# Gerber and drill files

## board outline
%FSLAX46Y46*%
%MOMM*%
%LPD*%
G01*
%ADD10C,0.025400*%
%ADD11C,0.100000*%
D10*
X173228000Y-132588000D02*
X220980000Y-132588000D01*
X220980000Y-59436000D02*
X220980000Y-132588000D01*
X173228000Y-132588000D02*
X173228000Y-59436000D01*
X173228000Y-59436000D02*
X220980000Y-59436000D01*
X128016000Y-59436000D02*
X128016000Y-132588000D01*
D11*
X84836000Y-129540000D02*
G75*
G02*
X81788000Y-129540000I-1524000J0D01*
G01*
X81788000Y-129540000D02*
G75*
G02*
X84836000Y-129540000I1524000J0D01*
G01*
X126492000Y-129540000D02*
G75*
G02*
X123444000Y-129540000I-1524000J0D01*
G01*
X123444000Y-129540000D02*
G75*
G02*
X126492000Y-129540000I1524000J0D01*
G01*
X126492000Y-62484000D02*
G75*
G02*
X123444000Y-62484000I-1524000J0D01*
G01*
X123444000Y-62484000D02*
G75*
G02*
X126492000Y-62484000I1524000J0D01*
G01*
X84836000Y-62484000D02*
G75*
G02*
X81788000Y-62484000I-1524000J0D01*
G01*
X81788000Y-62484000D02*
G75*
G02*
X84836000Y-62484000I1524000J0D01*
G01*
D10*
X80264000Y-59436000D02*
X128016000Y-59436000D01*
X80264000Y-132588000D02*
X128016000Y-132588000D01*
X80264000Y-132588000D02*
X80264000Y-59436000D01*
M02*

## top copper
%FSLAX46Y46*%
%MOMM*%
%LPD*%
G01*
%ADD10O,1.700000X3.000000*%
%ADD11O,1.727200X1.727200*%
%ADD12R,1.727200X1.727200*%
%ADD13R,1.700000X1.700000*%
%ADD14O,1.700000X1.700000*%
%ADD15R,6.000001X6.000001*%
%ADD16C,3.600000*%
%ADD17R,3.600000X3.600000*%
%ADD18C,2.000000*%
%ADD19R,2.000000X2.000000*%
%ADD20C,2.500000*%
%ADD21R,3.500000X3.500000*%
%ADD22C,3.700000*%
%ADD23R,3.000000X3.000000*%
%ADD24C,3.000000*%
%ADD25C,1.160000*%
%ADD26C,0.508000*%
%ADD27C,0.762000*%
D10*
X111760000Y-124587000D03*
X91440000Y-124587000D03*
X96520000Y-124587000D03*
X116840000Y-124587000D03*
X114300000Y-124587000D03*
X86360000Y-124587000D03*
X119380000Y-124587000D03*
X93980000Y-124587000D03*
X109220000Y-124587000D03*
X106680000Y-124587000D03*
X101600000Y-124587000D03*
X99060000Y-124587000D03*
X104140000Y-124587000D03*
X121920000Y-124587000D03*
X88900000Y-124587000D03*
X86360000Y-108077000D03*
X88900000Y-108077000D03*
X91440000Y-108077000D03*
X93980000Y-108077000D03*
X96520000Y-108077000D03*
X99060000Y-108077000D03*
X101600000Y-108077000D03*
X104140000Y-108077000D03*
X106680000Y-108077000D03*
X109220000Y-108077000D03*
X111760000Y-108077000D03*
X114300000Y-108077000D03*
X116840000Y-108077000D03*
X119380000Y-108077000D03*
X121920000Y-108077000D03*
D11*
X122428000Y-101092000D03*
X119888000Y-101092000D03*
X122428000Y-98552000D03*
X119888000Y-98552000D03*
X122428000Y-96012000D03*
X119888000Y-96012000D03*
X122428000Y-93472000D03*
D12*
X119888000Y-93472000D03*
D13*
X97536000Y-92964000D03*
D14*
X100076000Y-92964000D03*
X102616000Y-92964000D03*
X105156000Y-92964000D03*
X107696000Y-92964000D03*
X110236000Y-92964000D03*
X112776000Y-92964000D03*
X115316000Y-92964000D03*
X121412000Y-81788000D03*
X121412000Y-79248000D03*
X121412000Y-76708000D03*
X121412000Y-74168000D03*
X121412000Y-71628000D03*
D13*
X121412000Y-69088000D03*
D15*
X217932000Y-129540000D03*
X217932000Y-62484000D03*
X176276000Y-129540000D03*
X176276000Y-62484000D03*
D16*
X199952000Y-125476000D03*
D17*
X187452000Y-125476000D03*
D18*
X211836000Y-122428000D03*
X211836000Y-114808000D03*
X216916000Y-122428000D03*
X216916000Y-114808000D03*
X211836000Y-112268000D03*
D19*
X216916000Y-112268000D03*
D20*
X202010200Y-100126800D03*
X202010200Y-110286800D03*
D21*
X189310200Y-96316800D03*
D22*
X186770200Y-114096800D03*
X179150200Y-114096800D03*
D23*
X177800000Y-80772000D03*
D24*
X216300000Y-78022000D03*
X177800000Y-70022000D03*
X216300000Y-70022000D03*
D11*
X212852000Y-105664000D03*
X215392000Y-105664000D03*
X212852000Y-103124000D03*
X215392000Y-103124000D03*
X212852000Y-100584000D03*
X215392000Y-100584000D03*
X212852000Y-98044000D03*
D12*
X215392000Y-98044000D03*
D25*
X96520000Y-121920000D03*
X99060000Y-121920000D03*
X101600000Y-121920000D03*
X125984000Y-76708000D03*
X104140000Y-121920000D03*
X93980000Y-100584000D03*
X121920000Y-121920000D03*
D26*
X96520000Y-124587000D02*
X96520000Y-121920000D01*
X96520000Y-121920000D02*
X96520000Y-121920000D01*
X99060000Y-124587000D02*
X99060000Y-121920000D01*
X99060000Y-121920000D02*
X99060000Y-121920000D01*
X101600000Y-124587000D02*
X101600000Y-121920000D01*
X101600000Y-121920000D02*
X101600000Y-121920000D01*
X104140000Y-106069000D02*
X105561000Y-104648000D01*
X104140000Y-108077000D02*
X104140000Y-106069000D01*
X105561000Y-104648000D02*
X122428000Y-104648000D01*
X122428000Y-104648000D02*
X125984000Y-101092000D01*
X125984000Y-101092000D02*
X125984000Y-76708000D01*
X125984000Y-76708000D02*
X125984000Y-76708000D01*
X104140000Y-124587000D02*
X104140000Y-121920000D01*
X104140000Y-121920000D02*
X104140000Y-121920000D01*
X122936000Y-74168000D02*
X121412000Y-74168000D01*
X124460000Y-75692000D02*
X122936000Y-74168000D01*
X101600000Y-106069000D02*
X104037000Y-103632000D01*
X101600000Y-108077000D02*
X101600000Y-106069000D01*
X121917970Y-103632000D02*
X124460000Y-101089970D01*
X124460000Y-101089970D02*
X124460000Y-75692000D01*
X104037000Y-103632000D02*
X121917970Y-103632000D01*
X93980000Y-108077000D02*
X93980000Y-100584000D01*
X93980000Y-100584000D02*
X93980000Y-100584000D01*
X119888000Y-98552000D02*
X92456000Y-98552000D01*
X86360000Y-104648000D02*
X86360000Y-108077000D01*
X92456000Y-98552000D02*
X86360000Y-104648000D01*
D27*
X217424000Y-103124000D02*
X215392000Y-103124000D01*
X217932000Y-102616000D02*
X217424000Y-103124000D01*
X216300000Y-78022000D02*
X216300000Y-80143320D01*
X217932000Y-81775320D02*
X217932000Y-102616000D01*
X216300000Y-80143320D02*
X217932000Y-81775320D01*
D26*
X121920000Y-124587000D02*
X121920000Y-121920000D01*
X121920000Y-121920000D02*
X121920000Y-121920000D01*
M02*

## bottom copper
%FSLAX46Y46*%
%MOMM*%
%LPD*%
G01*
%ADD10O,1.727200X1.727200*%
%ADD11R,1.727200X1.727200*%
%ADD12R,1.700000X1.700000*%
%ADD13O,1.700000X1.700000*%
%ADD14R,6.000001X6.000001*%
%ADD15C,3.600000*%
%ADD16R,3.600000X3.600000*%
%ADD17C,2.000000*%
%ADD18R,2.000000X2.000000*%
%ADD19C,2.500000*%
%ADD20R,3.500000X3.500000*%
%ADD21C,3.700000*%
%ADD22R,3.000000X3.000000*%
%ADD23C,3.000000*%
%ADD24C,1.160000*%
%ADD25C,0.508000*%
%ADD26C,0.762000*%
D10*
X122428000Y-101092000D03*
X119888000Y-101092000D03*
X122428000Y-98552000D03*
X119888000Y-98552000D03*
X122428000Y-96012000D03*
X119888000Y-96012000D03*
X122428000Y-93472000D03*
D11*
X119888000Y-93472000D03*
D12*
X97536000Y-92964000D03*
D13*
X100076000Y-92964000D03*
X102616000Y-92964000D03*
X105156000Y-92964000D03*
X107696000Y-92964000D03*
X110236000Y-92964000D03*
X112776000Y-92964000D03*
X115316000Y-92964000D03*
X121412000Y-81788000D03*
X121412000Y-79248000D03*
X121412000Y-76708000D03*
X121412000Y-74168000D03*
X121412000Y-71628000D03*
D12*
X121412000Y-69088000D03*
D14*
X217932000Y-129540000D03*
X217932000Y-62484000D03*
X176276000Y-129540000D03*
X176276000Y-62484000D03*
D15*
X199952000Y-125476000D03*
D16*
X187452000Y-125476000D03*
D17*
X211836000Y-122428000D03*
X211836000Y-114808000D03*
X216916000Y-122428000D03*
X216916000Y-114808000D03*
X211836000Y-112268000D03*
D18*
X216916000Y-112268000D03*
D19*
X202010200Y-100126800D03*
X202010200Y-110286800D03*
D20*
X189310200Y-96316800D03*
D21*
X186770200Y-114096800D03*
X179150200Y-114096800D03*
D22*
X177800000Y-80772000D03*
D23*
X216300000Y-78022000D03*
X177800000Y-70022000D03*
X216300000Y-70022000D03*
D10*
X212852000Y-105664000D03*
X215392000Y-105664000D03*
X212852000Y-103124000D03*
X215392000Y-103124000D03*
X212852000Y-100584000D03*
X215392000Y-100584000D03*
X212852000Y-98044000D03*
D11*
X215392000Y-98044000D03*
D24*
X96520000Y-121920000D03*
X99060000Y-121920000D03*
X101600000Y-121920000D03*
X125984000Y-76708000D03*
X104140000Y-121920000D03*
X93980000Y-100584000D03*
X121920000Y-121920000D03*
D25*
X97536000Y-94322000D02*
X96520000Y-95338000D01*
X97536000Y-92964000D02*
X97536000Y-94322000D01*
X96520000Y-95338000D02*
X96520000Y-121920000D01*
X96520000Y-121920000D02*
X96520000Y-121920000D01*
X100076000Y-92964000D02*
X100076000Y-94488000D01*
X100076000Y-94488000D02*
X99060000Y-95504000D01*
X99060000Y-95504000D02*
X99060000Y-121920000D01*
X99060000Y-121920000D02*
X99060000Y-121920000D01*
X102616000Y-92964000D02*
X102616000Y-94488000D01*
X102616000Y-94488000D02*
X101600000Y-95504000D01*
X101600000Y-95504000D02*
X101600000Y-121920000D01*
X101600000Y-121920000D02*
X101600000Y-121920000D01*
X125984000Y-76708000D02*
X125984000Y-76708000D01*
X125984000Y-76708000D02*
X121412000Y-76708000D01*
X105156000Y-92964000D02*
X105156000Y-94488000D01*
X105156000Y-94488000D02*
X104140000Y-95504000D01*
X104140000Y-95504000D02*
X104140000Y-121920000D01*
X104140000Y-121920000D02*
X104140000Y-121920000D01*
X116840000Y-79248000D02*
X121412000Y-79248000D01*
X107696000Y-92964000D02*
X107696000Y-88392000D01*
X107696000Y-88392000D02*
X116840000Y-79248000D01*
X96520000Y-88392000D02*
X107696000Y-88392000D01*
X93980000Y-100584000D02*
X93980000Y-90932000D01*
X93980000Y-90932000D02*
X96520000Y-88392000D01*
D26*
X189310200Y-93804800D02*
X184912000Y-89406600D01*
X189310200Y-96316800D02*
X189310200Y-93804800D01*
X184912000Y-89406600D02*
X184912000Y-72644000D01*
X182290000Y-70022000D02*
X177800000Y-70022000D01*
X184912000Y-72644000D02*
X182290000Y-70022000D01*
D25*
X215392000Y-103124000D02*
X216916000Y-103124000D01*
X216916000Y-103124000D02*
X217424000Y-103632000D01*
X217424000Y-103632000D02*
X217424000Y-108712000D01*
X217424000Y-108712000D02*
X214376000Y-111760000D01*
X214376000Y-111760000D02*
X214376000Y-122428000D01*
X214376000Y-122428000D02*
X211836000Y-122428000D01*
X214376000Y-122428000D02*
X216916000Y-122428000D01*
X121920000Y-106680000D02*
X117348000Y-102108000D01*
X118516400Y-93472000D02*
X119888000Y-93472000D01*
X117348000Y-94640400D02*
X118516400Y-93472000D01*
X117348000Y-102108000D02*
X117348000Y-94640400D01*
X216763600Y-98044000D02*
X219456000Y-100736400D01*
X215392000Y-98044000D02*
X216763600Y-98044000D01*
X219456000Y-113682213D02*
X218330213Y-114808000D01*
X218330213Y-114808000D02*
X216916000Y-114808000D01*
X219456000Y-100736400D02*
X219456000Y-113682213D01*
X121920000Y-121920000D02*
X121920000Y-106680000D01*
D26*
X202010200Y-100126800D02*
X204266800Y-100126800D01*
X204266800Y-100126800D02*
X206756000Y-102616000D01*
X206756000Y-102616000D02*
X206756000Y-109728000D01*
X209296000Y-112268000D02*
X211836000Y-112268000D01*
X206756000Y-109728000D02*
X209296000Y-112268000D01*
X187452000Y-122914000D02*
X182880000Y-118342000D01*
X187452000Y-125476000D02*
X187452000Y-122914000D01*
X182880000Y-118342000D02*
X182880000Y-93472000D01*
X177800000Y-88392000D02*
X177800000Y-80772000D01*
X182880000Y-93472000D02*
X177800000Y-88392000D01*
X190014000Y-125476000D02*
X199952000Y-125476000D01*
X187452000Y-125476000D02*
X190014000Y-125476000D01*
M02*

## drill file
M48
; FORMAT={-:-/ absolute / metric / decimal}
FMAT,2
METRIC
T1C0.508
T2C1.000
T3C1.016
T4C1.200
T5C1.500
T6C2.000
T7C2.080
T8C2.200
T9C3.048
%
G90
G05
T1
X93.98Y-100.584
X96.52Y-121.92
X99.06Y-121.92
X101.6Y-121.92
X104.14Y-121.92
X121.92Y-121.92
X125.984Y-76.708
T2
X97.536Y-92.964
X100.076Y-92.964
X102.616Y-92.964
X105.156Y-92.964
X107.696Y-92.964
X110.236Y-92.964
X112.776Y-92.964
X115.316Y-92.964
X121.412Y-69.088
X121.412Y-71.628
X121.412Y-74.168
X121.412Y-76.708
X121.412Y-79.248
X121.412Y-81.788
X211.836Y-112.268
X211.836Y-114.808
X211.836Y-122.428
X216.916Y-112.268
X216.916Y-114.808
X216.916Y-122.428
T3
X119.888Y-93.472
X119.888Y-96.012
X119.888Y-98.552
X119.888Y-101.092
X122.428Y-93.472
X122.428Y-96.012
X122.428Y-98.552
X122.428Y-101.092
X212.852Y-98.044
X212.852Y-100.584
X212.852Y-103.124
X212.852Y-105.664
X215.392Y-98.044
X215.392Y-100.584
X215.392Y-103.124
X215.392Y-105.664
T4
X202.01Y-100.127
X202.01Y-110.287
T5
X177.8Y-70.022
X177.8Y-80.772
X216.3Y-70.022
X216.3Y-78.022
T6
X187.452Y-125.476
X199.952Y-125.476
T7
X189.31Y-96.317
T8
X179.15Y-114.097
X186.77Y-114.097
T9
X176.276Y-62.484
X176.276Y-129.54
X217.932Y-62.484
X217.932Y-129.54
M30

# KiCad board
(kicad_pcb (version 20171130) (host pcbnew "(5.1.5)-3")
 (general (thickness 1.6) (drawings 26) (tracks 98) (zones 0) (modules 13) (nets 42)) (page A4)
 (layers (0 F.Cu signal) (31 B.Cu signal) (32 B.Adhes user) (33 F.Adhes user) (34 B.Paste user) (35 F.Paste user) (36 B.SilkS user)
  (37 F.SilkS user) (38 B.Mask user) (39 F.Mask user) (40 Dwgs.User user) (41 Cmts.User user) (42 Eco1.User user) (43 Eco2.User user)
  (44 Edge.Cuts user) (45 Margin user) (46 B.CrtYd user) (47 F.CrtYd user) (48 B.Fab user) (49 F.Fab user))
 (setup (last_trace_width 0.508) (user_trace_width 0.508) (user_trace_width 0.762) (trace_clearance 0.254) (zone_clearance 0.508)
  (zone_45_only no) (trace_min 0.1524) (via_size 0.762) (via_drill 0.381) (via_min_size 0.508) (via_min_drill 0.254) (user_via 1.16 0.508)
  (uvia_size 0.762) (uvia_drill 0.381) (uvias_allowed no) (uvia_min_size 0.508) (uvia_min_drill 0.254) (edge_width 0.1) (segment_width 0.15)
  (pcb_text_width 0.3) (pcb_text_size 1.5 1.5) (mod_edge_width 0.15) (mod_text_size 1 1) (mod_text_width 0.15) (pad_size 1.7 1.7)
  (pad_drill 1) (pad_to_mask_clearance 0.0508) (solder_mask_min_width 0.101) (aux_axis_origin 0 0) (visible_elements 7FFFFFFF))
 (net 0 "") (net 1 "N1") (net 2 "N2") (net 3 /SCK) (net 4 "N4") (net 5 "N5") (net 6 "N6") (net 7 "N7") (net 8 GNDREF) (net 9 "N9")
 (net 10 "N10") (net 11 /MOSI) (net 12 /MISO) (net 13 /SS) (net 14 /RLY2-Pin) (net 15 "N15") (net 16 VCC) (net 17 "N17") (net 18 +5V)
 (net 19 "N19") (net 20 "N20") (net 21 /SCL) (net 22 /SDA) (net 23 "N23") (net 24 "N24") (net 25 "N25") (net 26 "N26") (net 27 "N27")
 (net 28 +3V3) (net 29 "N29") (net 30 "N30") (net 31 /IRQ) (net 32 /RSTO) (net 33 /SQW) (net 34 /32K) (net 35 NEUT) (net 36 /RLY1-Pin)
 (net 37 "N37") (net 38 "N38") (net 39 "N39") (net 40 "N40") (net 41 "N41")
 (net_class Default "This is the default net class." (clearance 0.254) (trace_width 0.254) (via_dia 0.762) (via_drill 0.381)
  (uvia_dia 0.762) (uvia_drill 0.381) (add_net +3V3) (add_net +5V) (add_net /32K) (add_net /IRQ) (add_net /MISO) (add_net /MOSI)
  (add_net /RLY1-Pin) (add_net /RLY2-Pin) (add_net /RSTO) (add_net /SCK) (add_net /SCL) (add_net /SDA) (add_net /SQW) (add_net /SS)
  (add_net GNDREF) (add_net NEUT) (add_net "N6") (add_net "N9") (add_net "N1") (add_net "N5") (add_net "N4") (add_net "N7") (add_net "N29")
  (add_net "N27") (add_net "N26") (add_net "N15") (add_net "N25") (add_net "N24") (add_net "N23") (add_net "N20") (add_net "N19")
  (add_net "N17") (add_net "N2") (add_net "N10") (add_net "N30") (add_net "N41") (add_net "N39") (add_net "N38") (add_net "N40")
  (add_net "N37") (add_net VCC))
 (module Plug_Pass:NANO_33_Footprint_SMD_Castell (layer F.Cu) (at 104.14 116.332)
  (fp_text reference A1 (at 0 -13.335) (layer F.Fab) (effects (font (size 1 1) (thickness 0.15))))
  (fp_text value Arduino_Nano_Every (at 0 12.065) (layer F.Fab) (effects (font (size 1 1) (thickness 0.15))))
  (pad 11 smd oval (at 7.62 8.255 90) (size 3 1.7) (layers F.Cu F.Mask) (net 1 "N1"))
  (pad 3 smd oval (at -12.7 8.255 90) (size 3 1.7) (layers F.Cu F.Mask) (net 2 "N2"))
  (pad 5 smd oval (at -7.62 8.255 90) (size 3 1.7) (layers F.Cu F.Mask) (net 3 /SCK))
  (pad 13 smd oval (at 12.7 8.255 90) (size 3 1.7) (layers F.Cu F.Mask) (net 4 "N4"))
  (pad 12 smd oval (at 10.16 8.255 90) (size 3 1.7) (layers F.Cu F.Mask) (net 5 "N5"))
  (pad 1 smd oval (at -17.78 8.255 90) (size 3 1.7) (layers F.Cu F.Mask) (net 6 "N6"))
  (pad 14 smd oval (at 15.24 8.255 90) (size 3 1.7) (layers F.Cu F.Mask) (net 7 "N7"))
  (pad 4 smd oval (at -10.16 8.255 90) (size 3 1.7) (layers F.Cu F.Mask) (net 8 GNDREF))
  (pad 10 smd oval (at 5.08 8.255 90) (size 3 1.7) (layers F.Cu F.Mask) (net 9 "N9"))
  (pad 9 smd oval (at 2.54 8.255 90) (size 3 1.7) (layers F.Cu F.Mask) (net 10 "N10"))
  (pad 7 smd oval (at -2.54 8.255 90) (size 3 1.7) (layers F.Cu F.Mask) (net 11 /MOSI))
  (pad 6 smd oval (at -5.08 8.255 90) (size 3 1.7) (layers F.Cu F.Mask) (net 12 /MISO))
  (pad 8 smd oval (at 0 8.255 90) (size 3 1.7) (layers F.Cu F.Mask) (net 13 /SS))
  (pad 15 smd oval (at 17.78 8.255 90) (size 3 1.7) (layers F.Cu F.Mask) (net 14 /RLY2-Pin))
  (pad 2 smd oval (at -15.24 8.255 90) (size 3 1.7) (layers F.Cu F.Mask) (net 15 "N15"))
  (pad 30 smd oval (at -17.78 -8.255 270) (size 3 1.7) (layers F.Cu F.Mask) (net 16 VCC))
  (pad 29 smd oval (at -15.24 -8.255 270) (size 3 1.7) (layers F.Cu F.Mask) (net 8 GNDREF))
  (pad 28 smd oval (at -12.7 -8.255 270) (size 3 1.7) (layers F.Cu F.Mask) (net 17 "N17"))
  (pad 27 smd oval (at -10.16 -8.255 270) (size 3 1.7) (layers F.Cu F.Mask) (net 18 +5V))
  (pad 26 smd oval (at -7.62 -8.255 270) (size 3 1.7) (layers F.Cu F.Mask) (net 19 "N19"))
  (pad 25 smd oval (at -5.08 -8.255 270) (size 3 1.7) (layers F.Cu F.Mask) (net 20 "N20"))
  (pad 24 smd oval (at -2.54 -8.255 270) (size 3 1.7) (layers F.Cu F.Mask) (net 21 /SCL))
  (pad 23 smd oval (at 0 -8.255 270) (size 3 1.7) (layers F.Cu F.Mask) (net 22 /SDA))
  (pad 22 smd oval (at 2.54 -8.255 270) (size 3 1.7) (layers F.Cu F.Mask) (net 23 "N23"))
  (pad 21 smd oval (at 5.08 -8.255 270) (size 3 1.7) (layers F.Cu F.Mask) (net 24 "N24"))
  (pad 20 smd oval (at 7.62 -8.255 270) (size 3 1.7) (layers F.Cu F.Mask) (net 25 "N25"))
  (pad 19 smd oval (at 10.16 -8.255 270) (size 3 1.7) (layers F.Cu F.Mask) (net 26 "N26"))
  (pad 18 smd oval (at 12.7 -8.255 270) (size 3 1.7) (layers F.Cu F.Mask) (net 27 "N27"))
  (pad 17 smd oval (at 15.24 -8.255 270) (size 3 1.7) (layers F.Cu F.Mask) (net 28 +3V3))
  (pad 16 smd oval (at 17.78 -8.255 270) (size 3 1.7) (layers F.Cu F.Mask) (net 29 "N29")))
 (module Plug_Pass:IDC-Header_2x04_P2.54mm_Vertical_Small (layer F.Cu) (at 119.888 93.472)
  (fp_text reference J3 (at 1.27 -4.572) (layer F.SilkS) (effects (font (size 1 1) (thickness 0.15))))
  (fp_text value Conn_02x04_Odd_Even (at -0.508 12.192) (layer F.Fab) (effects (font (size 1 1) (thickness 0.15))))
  (pad 8 thru_hole oval (at 2.54 7.62) (size 1.7272 1.7272) (drill 1.016) (layers *.Cu *.Mask) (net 8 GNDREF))
  (pad 7 thru_hole oval (at 0 7.62) (size 1.7272 1.7272) (drill 1.016) (layers *.Cu *.Mask) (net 8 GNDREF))
  (pad 6 thru_hole oval (at 2.54 5.08) (size 1.7272 1.7272) (drill 1.016) (layers *.Cu *.Mask) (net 8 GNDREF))
  (pad 5 thru_hole oval (at 0 5.08) (size 1.7272 1.7272) (drill 1.016) (layers *.Cu *.Mask) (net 16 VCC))
  (pad 4 thru_hole oval (at 2.54 2.54) (size 1.7272 1.7272) (drill 1.016) (layers *.Cu *.Mask) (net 8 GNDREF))
  (pad 3 thru_hole oval (at 0 2.54) (size 1.7272 1.7272) (drill 1.016) (layers *.Cu *.Mask) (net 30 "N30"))
  (pad 2 thru_hole oval (at 2.54 0) (size 1.7272 1.7272) (drill 1.016) (layers *.Cu *.Mask) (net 8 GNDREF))
  (pad 1 thru_hole rect (at 0 0) (size 1.7272 1.7272) (drill 1.016) (layers *.Cu *.Mask) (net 14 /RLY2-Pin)))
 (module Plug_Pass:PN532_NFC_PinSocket (layer F.Cu) (at 97.536 92.964 90)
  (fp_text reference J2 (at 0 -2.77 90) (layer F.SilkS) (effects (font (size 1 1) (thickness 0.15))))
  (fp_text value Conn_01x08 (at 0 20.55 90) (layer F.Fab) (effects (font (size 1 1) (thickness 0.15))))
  (pad 1 thru_hole rect (at 0 0 90) (size 1.7 1.7) (drill 1) (layers *.Cu *.Mask) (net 3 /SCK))
  (pad 2 thru_hole oval (at 0 2.54 90) (size 1.7 1.7) (drill 1) (layers *.Cu *.Mask) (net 12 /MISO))
  (pad 3 thru_hole oval (at 0 5.08 90) (size 1.7 1.7) (drill 1) (layers *.Cu *.Mask) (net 11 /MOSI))
  (pad 4 thru_hole oval (at 0 7.62 90) (size 1.7 1.7) (drill 1) (layers *.Cu *.Mask) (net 13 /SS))
  (pad 5 thru_hole oval (at 0 10.16 90) (size 1.7 1.7) (drill 1) (layers *.Cu *.Mask) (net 18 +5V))
  (pad 6 thru_hole oval (at 0 12.7 90) (size 1.7 1.7) (drill 1) (layers *.Cu *.Mask) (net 8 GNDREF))
  (pad 7 thru_hole oval (at 0 15.24 90) (size 1.7 1.7) (drill 1) (layers *.Cu *.Mask) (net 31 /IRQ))
  (pad 8 thru_hole oval (at 0 17.78 90) (size 1.7 1.7) (drill 1) (layers *.Cu *.Mask) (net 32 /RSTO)))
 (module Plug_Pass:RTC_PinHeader (layer F.Cu) (at 121.412 69.088)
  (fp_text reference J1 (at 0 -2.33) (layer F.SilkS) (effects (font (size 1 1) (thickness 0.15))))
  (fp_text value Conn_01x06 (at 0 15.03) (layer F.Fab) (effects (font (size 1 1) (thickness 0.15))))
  (pad 6 thru_hole oval (at 0 12.7) (size 1.7 1.7) (drill 1) (layers *.Cu *.Mask) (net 8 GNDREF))
  (pad 5 thru_hole oval (at 0 10.16) (size 1.7 1.7) (drill 1) (layers *.Cu *.Mask) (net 18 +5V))
  (pad 4 thru_hole oval (at 0 7.62) (size 1.7 1.7) (drill 1) (layers *.Cu *.Mask) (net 22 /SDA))
  (pad 3 thru_hole oval (at 0 5.08) (size 1.7 1.7) (drill 1) (layers *.Cu *.Mask) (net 21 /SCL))
  (pad 2 thru_hole oval (at 0 2.54) (size 1.7 1.7) (drill 1) (layers *.Cu *.Mask) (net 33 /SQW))
  (pad 1 thru_hole rect (at 0 0) (size 1.7 1.7) (drill 1) (layers *.Cu *.Mask) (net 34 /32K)))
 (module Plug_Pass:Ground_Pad (layer F.Cu) (at 217.932 129.54)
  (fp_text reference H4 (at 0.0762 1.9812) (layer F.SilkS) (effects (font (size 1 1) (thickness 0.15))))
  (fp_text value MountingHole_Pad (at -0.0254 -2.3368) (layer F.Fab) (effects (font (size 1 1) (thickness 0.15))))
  (pad 1 thru_hole rect (at 0 0) (size 6.000001 6.000001) (drill 3.048) (layers *.Cu *.Mask) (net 8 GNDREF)))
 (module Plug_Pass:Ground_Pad (layer F.Cu) (at 217.932 62.484)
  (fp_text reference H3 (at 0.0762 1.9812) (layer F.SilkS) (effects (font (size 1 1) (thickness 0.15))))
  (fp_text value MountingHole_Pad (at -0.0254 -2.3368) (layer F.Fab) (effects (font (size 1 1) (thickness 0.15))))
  (pad 1 thru_hole rect (at 0 0) (size 6.000001 6.000001) (drill 3.048) (layers *.Cu *.Mask) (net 8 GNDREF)))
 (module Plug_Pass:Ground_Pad (layer F.Cu) (at 176.276 129.54)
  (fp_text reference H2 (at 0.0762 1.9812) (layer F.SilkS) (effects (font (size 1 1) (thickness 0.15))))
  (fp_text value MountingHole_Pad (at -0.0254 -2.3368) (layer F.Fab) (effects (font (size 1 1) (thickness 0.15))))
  (pad 1 thru_hole rect (at 0 0) (size 6.000001 6.000001) (drill 3.048) (layers *.Cu *.Mask) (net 8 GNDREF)))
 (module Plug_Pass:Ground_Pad (layer F.Cu) (at 176.276 62.484)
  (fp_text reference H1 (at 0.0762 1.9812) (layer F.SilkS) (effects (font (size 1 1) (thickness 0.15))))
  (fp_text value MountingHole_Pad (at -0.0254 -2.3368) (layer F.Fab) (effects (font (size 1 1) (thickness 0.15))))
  (pad 1 thru_hole rect (at 0 0) (size 6.000001 6.000001) (drill 3.048) (layers *.Cu *.Mask) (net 8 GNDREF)))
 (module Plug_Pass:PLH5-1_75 (layer B.Cu) (at 187.452 125.476 270)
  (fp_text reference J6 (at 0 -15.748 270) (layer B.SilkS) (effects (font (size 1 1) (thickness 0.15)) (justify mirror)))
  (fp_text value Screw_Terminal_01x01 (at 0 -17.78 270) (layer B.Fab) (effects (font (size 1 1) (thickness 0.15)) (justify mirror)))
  (pad 1 thru_hole circle (at 0 -12.5 270) (size 3.6 3.6) (drill 2) (layers *.Cu *.Mask) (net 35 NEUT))
  (pad 1 thru_hole rect (at 0 0 270) (size 3.6 3.6) (drill 2) (layers *.Cu *.Mask) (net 35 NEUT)))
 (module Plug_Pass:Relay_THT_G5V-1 (layer B.Cu) (at 216.916 112.268 270)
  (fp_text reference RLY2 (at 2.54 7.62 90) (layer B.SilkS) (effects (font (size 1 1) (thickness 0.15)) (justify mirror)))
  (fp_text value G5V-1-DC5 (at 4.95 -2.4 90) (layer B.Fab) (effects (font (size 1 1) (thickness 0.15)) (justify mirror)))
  (pad 6 thru_hole circle (at 10.16 5.08 270) (size 2 2) (drill 1) (layers *.Cu *.Mask) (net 16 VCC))
  (pad 9 thru_hole circle (at 2.54 5.08 270) (size 2 2) (drill 1) (layers *.Cu *.Mask) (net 8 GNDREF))
  (pad 5 thru_hole circle (at 10.16 0 270) (size 2 2) (drill 1) (layers *.Cu *.Mask) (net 16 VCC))
  (pad 2 thru_hole circle (at 2.54 0 270) (size 2 2) (drill 1) (layers *.Cu *.Mask) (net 14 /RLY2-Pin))
  (pad 10 thru_hole circle (at 0 5.08 270) (size 2 2) (drill 1) (layers *.Cu *.Mask) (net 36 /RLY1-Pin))
  (pad 1 thru_hole rect (at 0 0 270) (size 2 2) (drill 1) (layers *.Cu *.Mask) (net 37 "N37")))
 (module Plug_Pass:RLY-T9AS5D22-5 (layer B.Cu) (at 175.768 92.964 270)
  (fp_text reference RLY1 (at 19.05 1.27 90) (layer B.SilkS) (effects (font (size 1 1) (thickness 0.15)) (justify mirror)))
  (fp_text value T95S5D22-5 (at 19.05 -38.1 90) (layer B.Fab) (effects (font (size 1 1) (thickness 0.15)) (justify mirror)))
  (pad 5 thru_hole circle (at 7.1628 -26.2422 270) (size 2.5 2.5) (drill 1.2) (layers *.Cu *.Mask) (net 36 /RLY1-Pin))
  (pad 2 thru_hole circle (at 17.3228 -26.2422 270) (size 2.5 2.5) (drill 1.2) (layers *.Cu *.Mask) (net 8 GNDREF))
  (pad 1 thru_hole rect (at 3.3528 -13.5422 270) (size 3.5 3.5) (drill 2.08) (layers *.Cu *.Mask) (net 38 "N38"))
  (pad 3 thru_hole circle (at 21.1328 -11.0022 270) (size 3.7 3.7) (drill 2.2) (layers *.Cu *.Mask) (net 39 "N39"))
  (pad 4 thru_hole circle (at 21.1328 -3.3822 270) (size 3.7 3.7) (drill 2.2) (layers *.Cu *.Mask) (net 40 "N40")))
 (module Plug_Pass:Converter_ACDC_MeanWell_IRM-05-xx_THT (layer B.Cu) (at 177.8 80.772)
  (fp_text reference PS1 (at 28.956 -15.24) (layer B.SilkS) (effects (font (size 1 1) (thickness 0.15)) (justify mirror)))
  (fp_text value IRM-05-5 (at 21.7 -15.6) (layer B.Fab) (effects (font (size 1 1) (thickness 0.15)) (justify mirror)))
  (pad 1 thru_hole rect (at 0 0) (size 3 3) (drill 1.5) (layers *.Cu *.Mask) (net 35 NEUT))
  (pad 4 thru_hole circle (at 38.5 -2.75) (size 3 3) (drill 1.5) (layers *.Cu *.Mask) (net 16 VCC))
  (pad 2 thru_hole circle (at 0 -10.75) (size 3 3) (drill 1.5) (layers *.Cu *.Mask) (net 38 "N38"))
  (pad 3 thru_hole circle (at 38.5 -10.75) (size 3 3) (drill 1.5) (layers *.Cu *.Mask) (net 8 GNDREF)))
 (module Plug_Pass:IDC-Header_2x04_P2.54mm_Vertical (layer B.Cu) (at 215.392 98.044 180)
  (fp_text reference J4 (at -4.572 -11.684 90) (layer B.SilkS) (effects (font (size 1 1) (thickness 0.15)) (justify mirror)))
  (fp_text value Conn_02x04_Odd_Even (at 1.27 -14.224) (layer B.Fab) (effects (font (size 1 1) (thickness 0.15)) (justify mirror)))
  (pad 8 thru_hole oval (at 2.54 -7.62 180) (size 1.7272 1.7272) (drill 1.016) (layers *.Cu *.Mask) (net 8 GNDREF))
  (pad 7 thru_hole oval (at 0 -7.62 180) (size 1.7272 1.7272) (drill 1.016) (layers *.Cu *.Mask) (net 8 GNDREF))
  (pad 6 thru_hole oval (at 2.54 -5.08 180) (size 1.7272 1.7272) (drill 1.016) (layers *.Cu *.Mask) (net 8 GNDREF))
  (pad 5 thru_hole oval (at 0 -5.08 180) (size 1.7272 1.7272) (drill 1.016) (layers *.Cu *.Mask) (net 16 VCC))
  (pad 4 thru_hole oval (at 2.54 -2.54 180) (size 1.7272 1.7272) (drill 1.016) (layers *.Cu *.Mask) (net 8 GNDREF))
  (pad 3 thru_hole oval (at 0 -2.54 180) (size 1.7272 1.7272) (drill 1.016) (layers *.Cu *.Mask) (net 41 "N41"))
  (pad 2 thru_hole oval (at 2.54 0 180) (size 1.7272 1.7272) (drill 1.016) (layers *.Cu *.Mask) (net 8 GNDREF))
  (pad 1 thru_hole rect (at 0 0 180) (size 1.7272 1.7272) (drill 1.016) (layers *.Cu *.Mask) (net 14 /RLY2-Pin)))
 (gr_line (start 173.228 132.588) (end 220.98 132.588) (layer Edge.Cuts) (width 0.0254))
 (gr_line (start 220.98 59.436) (end 220.98 132.588) (layer Edge.Cuts) (width 0.0254))
 (gr_line (start 173.228 132.588) (end 173.228 59.436) (layer Edge.Cuts) (width 0.0254))
 (gr_line (start 173.228 59.436) (end 220.98 59.436) (layer Edge.Cuts) (width 0.0254))
 (gr_line (start 128.016 59.436) (end 128.016 132.588) (layer Edge.Cuts) (width 0.0254))
 (gr_circle (center 83.312 129.54) (end 84.836 129.54) (layer Edge.Cuts) (width 0.1))
 (gr_circle (center 124.968 129.54) (end 126.492 129.54) (layer Edge.Cuts) (width 0.1))
 (gr_circle (center 124.968 62.484) (end 126.492 62.484) (layer Edge.Cuts) (width 0.1))
 (gr_circle (center 83.312 62.484) (end 84.836 62.484) (layer Edge.Cuts) (width 0.1))
 (gr_line (start 80.264 59.436) (end 128.016 59.436) (layer Edge.Cuts) (width 0.0254))
 (gr_line (start 80.264 132.588) (end 128.016 132.588) (layer Edge.Cuts) (width 0.0254))
 (gr_line (start 80.264 132.588) (end 80.264 59.436) (layer Edge.Cuts) (width 0.0254))
 (segment (start 97.536 94.322) (end 96.52 95.338) (width 0.508) (layer B.Cu) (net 3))
 (segment (start 97.536 92.964) (end 97.536 94.322) (width 0.508) (layer B.Cu) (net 3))
 (segment (start 96.52 95.338) (end 96.52 121.92) (width 0.508) (layer B.Cu) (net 3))
 (segment (start 96.52 121.92) (end 96.52 121.92) (width 0.508) (layer B.Cu) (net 3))
 (segment (start 96.52 124.587) (end 96.52 121.92) (width 0.508) (layer F.Cu) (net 3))
 (segment (start 96.52 121.92) (end 96.52 121.92) (width 0.508) (layer F.Cu) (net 3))
 (via (at 96.52 121.92) (size 1.16) (drill 0.508) (layers F.Cu B.Cu) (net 3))
 (segment (start 100.076 92.964) (end 100.076 94.488) (width 0.508) (layer B.Cu) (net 12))
 (segment (start 100.076 94.488) (end 99.06 95.504) (width 0.508) (layer B.Cu) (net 12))
 (segment (start 99.06 95.504) (end 99.06 121.92) (width 0.508) (layer B.Cu) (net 12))
 (segment (start 99.06 121.92) (end 99.06 121.92) (width 0.508) (layer B.Cu) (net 12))
 (segment (start 99.06 124.587) (end 99.06 121.92) (width 0.508) (layer F.Cu) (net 12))
 (segment (start 99.06 121.92) (end 99.06 121.92) (width 0.508) (layer F.Cu) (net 12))
 (via (at 99.06 121.92) (size 1.16) (drill 0.508) (layers F.Cu B.Cu) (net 12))
 (segment (start 102.616 92.964) (end 102.616 94.488) (width 0.508) (layer B.Cu) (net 11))
 (segment (start 102.616 94.488) (end 101.6 95.504) (width 0.508) (layer B.Cu) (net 11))
 (segment (start 101.6 95.504) (end 101.6 121.92) (width 0.508) (layer B.Cu) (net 11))
 (segment (start 101.6 121.92) (end 101.6 121.92) (width 0.508) (layer B.Cu) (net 11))
 (segment (start 101.6 124.587) (end 101.6 121.92) (width 0.508) (layer F.Cu) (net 11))
 (segment (start 101.6 121.92) (end 101.6 121.92) (width 0.508) (layer F.Cu) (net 11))
 (via (at 101.6 121.92) (size 1.16) (drill 0.508) (layers F.Cu B.Cu) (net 11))
 (segment (start 104.14 106.069) (end 105.561 104.648) (width 0.508) (layer F.Cu) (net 22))
 (segment (start 104.14 108.077) (end 104.14 106.069) (width 0.508) (layer F.Cu) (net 22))
 (segment (start 105.561 104.648) (end 122.428 104.648) (width 0.508) (layer F.Cu) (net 22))
 (segment (start 122.428 104.648) (end 125.984 101.092) (width 0.508) (layer F.Cu) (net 22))
 (segment (start 125.984 101.092) (end 125.984 76.708) (width 0.508) (layer F.Cu) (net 22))
 (segment (start 125.984 76.708) (end 125.984 76.708) (width 0.508) (layer F.Cu) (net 22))
 (segment (start 125.984 76.708) (end 125.984 76.708) (width 0.508) (layer B.Cu) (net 22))
 (segment (start 125.984 76.708) (end 121.412 76.708) (width 0.508) (layer B.Cu) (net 22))
 (via (at 125.984 76.708) (size 1.16) (drill 0.508) (layers F.Cu B.Cu) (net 22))
 (segment (start 105.156 92.964) (end 105.156 94.488) (width 0.508) (layer B.Cu) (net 13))
 (segment (start 105.156 94.488) (end 104.14 95.504) (width 0.508) (layer B.Cu) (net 13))
 (segment (start 104.14 95.504) (end 104.14 121.92) (width 0.508) (layer B.Cu) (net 13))
 (segment (start 104.14 121.92) (end 104.14 121.92) (width 0.508) (layer B.Cu) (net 13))
 (segment (start 104.14 124.587) (end 104.14 121.92) (width 0.508) (layer F.Cu) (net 13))
 (segment (start 104.14 121.92) (end 104.14 121.92) (width 0.508) (layer F.Cu) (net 13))
 (via (at 104.14 121.92) (size 1.16) (drill 0.508) (layers F.Cu B.Cu) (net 13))
 (segment (start 122.936 74.168) (end 121.412 74.168) (width 0.508) (layer F.Cu) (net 21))
 (segment (start 124.46 75.692) (end 122.936 74.168) (width 0.508) (layer F.Cu) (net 21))
 (segment (start 101.6 106.069) (end 104.037 103.632) (width 0.508) (layer F.Cu) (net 21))
 (segment (start 101.6 108.077) (end 101.6 106.069) (width 0.508) (layer F.Cu) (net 21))
 (segment (start 121.91797 103.632) (end 124.46 101.08997) (width 0.508) (layer F.Cu) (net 21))
 (segment (start 124.46 101.08997) (end 124.46 75.692) (width 0.508) (layer F.Cu) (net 21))
 (segment (start 104.037 103.632) (end 121.91797 103.632) (width 0.508) (layer F.Cu) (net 21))
 (segment (start 116.84 79.248) (end 121.412 79.248) (width 0.508) (layer B.Cu) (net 18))
 (segment (start 107.696 92.964) (end 107.696 88.392) (width 0.508) (layer B.Cu) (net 18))
 (segment (start 107.696 88.392) (end 116.84 79.248) (width 0.508) (layer B.Cu) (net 18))
 (segment (start 93.98 108.077) (end 93.98 100.584) (width 0.508) (layer F.Cu) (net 18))
 (segment (start 93.98 100.584) (end 93.98 100.584) (width 0.508) (layer F.Cu) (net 18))
 (via (at 93.98 100.584) (size 1.16) (drill 0.508) (layers F.Cu B.Cu) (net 18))
 (segment (start 96.52 88.392) (end 107.696 88.392) (width 0.508) (layer B.Cu) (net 18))
 (segment (start 93.98 100.584) (end 93.98 90.932) (width 0.508) (layer B.Cu) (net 18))
 (segment (start 93.98 90.932) (end 96.52 88.392) (width 0.508) (layer B.Cu) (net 18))
 (segment (start 189.3102 93.8048) (end 184.912 89.4066) (width 0.762) (layer B.Cu) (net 38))
 (segment (start 189.3102 96.3168) (end 189.3102 93.8048) (width 0.762) (layer B.Cu) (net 38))
 (segment (start 184.912 89.4066) (end 184.912 72.644) (width 0.762) (layer B.Cu) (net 38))
 (segment (start 182.29 70.022) (end 177.8 70.022) (width 0.762) (layer B.Cu) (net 38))
 (segment (start 184.912 72.644) (end 182.29 70.022) (width 0.762) (layer B.Cu) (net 38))
 (segment (start 119.888 98.552) (end 92.456 98.552) (width 0.508) (layer F.Cu) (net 16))
 (segment (start 86.36 104.648) (end 86.36 108.077) (width 0.508) (layer F.Cu) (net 16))
 (segment (start 92.456 98.552) (end 86.36 104.648) (width 0.508) (layer F.Cu) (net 16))
 (segment (start 215.392 103.124) (end 216.916 103.124) (width 0.508) (layer B.Cu) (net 16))
 (segment (start 216.916 103.124) (end 217.424 103.632) (width 0.508) (layer B.Cu) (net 16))
 (segment (start 217.424 103.632) (end 217.424 108.712) (width 0.508) (layer B.Cu) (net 16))
 (segment (start 217.424 108.712) (end 214.376 111.76) (width 0.508) (layer B.Cu) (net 16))
 (segment (start 214.376 111.76) (end 214.376 122.428) (width 0.508) (layer B.Cu) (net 16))
 (segment (start 214.376 122.428) (end 211.836 122.428) (width 0.508) (layer B.Cu) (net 16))
 (segment (start 214.376 122.428) (end 216.916 122.428) (width 0.508) (layer B.Cu) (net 16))
 (segment (start 217.424 103.124) (end 215.392 103.124) (width 0.762) (layer F.Cu) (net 16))
 (segment (start 217.932 102.616) (end 217.424 103.124) (width 0.762) (layer F.Cu) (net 16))
 (segment (start 216.3 78.022) (end 216.3 80.14332) (width 0.762) (layer F.Cu) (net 16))
 (segment (start 217.932 81.77532) (end 217.932 102.616) (width 0.762) (layer F.Cu) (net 16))
 (segment (start 216.3 80.14332) (end 217.932 81.77532) (width 0.762) (layer F.Cu) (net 16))
 (segment (start 121.92 106.68) (end 117.348 102.108) (width 0.508) (layer B.Cu) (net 14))
 (segment (start 118.5164 93.472) (end 119.888 93.472) (width 0.508) (layer B.Cu) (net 14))
 (segment (start 117.348 94.6404) (end 118.5164 93.472) (width 0.508) (layer B.Cu) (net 14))
 (segment (start 117.348 102.108) (end 117.348 94.6404) (width 0.508) (layer B.Cu) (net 14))
 (segment (start 216.7636 98.044) (end 219.456 100.7364) (width 0.508) (layer B.Cu) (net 14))
 (segment (start 215.392 98.044) (end 216.7636 98.044) (width 0.508) (layer B.Cu) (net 14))
 (segment (start 219.456 113.682213) (end 218.330213 114.808) (width 0.508) (layer B.Cu) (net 14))
 (segment (start 218.330213 114.808) (end 216.916 114.808) (width 0.508) (layer B.Cu) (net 14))
 (segment (start 219.456 100.7364) (end 219.456 113.682213) (width 0.508) (layer B.Cu) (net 14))
 (segment (start 121.92 124.587) (end 121.92 121.92) (width 0.508) (layer F.Cu) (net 14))
 (segment (start 121.92 121.92) (end 121.92 121.92) (width 0.508) (layer F.Cu) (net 14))
 (via (at 121.92 121.92) (size 1.16) (drill 0.508) (layers F.Cu B.Cu) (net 14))
 (segment (start 121.92 121.92) (end 121.92 106.68) (width 0.508) (layer B.Cu) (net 14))
 (segment (start 202.0102 100.1268) (end 204.2668 100.1268) (width 0.762) (layer B.Cu) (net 36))
 (segment (start 204.2668 100.1268) (end 206.756 102.616) (width 0.762) (layer B.Cu) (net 36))
 (segment (start 206.756 102.616) (end 206.756 109.728) (width 0.762) (layer B.Cu) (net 36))
 (segment (start 209.296 112.268) (end 211.836 112.268) (width 0.762) (layer B.Cu) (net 36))
 (segment (start 206.756 109.728) (end 209.296 112.268) (width 0.762) (layer B.Cu) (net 36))
 (segment (start 187.452 122.914) (end 182.88 118.342) (width 0.762) (layer B.Cu) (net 35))
 (segment (start 187.452 125.476) (end 187.452 122.914) (width 0.762) (layer B.Cu) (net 35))
 (segment (start 182.88 118.342) (end 182.88 93.472) (width 0.762) (layer B.Cu) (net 35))
 (segment (start 177.8 88.392) (end 177.8 80.772) (width 0.762) (layer B.Cu) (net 35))
 (segment (start 182.88 93.472) (end 177.8 88.392) (width 0.762) (layer B.Cu) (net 35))
 (segment (start 190.014 125.476) (end 199.952 125.476) (width 0.762) (layer B.Cu) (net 35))
 (segment (start 187.452 125.476) (end 190.014 125.476) (width 0.762) (layer B.Cu) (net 35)))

